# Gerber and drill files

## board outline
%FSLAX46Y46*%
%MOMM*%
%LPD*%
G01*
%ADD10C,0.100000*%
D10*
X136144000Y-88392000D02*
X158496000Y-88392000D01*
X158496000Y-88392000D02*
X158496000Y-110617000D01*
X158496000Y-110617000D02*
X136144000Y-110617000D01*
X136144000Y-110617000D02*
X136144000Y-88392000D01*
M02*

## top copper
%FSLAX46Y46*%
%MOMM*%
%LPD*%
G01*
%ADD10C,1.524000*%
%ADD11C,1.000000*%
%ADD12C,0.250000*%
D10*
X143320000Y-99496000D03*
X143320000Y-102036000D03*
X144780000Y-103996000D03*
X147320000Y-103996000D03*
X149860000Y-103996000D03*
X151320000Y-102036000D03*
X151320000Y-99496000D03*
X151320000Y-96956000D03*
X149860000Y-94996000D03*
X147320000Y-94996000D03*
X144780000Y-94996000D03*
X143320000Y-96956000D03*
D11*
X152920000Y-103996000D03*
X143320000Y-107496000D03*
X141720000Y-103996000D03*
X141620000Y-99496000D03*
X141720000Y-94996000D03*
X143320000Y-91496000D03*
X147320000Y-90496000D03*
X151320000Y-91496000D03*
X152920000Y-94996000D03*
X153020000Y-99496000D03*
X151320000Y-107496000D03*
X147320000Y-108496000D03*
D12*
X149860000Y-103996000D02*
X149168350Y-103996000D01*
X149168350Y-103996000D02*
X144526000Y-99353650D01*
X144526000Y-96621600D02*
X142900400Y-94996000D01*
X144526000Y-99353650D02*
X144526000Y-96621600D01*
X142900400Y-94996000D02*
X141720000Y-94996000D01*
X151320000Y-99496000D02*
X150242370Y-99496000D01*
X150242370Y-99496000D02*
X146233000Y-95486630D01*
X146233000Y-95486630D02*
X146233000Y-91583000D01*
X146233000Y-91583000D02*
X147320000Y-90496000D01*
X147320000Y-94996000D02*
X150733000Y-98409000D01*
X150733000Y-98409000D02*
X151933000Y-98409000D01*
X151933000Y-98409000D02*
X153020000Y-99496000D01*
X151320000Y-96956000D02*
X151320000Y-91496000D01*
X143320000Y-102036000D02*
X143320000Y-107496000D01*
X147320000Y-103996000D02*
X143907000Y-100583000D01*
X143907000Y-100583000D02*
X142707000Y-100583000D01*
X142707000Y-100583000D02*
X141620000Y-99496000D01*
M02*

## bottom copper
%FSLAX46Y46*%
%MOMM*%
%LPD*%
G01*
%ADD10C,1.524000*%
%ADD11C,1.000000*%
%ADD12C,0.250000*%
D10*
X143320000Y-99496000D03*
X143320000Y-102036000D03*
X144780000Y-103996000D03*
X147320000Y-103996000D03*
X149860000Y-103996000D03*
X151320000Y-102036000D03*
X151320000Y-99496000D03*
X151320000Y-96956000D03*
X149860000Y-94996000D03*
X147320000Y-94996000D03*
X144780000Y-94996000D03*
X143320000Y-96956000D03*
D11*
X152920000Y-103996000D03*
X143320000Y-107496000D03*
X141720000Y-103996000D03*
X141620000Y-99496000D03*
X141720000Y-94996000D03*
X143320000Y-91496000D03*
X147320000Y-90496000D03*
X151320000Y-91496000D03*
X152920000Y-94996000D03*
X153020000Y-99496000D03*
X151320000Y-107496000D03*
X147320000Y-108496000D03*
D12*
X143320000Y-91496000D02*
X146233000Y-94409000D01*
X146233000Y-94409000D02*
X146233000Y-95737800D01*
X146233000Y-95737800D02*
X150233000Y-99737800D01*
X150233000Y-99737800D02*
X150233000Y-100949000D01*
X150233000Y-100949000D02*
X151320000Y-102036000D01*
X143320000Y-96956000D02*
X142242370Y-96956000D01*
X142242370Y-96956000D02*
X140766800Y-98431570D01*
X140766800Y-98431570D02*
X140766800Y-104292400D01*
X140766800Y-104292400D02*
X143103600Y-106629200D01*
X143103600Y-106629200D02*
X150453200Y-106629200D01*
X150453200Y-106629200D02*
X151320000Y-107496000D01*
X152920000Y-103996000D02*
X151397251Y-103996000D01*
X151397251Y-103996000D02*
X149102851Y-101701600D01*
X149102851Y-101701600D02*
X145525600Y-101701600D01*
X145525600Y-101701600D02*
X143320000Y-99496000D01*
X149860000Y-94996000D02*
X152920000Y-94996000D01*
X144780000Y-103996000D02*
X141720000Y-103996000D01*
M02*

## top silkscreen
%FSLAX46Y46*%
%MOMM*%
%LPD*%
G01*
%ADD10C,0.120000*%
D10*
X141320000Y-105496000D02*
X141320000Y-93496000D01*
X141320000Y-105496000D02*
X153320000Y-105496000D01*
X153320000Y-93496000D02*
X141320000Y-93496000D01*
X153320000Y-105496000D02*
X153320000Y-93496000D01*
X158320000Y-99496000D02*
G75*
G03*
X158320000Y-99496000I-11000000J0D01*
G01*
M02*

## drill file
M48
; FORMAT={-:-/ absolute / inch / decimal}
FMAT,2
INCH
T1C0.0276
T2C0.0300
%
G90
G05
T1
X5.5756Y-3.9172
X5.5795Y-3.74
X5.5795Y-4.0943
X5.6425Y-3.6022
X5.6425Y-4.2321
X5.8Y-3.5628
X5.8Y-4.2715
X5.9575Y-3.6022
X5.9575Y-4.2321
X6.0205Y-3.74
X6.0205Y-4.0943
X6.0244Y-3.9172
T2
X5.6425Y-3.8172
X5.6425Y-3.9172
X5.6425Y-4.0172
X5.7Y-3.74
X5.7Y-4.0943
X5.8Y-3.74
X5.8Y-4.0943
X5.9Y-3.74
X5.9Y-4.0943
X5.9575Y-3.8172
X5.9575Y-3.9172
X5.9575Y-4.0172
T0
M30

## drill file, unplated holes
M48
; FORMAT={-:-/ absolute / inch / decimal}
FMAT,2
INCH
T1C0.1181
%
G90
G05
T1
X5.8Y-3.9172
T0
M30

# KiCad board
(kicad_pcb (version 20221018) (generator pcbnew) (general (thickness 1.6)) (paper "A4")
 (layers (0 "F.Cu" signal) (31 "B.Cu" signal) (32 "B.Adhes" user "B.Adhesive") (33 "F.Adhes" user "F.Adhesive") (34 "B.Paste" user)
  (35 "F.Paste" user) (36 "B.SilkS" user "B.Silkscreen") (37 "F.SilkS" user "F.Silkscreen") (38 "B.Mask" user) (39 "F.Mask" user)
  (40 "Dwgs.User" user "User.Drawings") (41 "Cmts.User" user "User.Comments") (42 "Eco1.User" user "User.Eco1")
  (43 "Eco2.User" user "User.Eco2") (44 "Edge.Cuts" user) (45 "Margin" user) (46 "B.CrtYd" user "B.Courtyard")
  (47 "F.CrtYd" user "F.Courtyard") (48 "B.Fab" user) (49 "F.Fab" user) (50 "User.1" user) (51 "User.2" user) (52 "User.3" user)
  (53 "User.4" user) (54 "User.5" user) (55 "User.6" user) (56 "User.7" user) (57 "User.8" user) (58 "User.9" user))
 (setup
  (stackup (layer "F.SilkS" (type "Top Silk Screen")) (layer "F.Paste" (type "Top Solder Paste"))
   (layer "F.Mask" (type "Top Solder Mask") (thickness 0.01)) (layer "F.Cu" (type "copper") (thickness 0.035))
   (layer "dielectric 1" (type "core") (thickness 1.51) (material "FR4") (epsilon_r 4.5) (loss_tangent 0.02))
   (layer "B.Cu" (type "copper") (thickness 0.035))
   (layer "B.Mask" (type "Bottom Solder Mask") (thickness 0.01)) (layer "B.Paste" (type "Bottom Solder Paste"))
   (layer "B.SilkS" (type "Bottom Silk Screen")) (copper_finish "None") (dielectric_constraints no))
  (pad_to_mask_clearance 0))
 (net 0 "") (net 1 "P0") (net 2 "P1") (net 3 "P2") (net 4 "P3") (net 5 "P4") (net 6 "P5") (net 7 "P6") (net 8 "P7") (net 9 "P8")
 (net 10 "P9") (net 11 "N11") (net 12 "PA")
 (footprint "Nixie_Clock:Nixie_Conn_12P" (layer "F.Cu") (at 147.32 99.496)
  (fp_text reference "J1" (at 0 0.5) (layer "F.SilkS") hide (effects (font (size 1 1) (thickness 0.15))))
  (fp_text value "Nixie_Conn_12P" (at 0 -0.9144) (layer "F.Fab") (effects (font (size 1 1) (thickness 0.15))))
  (fp_line (start -6 6) (end -6 -6) (stroke (width 0.12) (type solid)) (layer "F.SilkS"))
  (fp_line (start -6 6) (end 6 6) (stroke (width 0.12) (type solid)) (layer "F.SilkS"))
  (fp_line (start 6 -6) (end -6 -6) (stroke (width 0.12) (type solid)) (layer "F.SilkS"))
  (fp_line (start 6 6) (end 6 -6) (stroke (width 0.12) (type solid)) (layer "F.SilkS"))
  (pad "0" thru_hole circle (at -4 0) (size 1.524 1.524) (drill 0.762) (layers "*.Cu" "*.Mask") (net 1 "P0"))
  (pad "1" thru_hole circle (at -4 2.54) (size 1.524 1.524) (drill 0.762) (layers "*.Cu" "*.Mask") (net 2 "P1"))
  (pad "2" thru_hole circle (at -2.54 4.5) (size 1.524 1.524) (drill 0.762) (layers "*.Cu" "*.Mask") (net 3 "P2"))
  (pad "3" thru_hole circle (at 0 4.5) (size 1.524 1.524) (drill 0.762) (layers "*.Cu" "*.Mask") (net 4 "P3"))
  (pad "4" thru_hole circle (at 2.54 4.5) (size 1.524 1.524) (drill 0.762) (layers "*.Cu" "*.Mask") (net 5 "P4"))
  (pad "5" thru_hole circle (at 4 2.54) (size 1.524 1.524) (drill 0.762) (layers "*.Cu" "*.Mask") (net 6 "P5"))
  (pad "6" thru_hole circle (at 4 0) (size 1.524 1.524) (drill 0.762) (layers "*.Cu" "*.Mask") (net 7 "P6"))
  (pad "7" thru_hole circle (at 4 -2.54) (size 1.524 1.524) (drill 0.762) (layers "*.Cu" "*.Mask") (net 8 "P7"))
  (pad "8" thru_hole circle (at 2.54 -4.5) (size 1.524 1.524) (drill 0.762) (layers "*.Cu" "*.Mask") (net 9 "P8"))
  (pad "9" thru_hole circle (at 0 -4.5) (size 1.524 1.524) (drill 0.762) (layers "*.Cu" "*.Mask") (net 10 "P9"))
  (pad "10" thru_hole circle (at -2.54 -4.5) (size 1.524 1.524) (drill 0.762) (layers "*.Cu" "*.Mask") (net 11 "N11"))
  (pad "A" thru_hole circle (at -4 -2.54) (size 1.524 1.524) (drill 0.762) (layers "*.Cu" "*.Mask") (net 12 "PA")))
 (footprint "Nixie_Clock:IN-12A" (layer "F.Cu") (at 147.32 99.496)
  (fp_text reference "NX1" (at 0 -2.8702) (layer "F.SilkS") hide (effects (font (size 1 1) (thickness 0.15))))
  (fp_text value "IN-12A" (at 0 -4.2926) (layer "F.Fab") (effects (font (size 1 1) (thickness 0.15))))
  (fp_circle (center 0 0) (end 11 0) (stroke (width 0.12) (type solid)) (fill none) (layer "F.SilkS"))
  (pad "" np_thru_hole circle (at 0 0) (size 3 3) (drill 3) (layers "*.Cu" "*.Mask"))
  (pad "0" thru_hole circle (at 5.6 4.5) (size 1 1) (drill 0.7) (layers "*.Cu" "*.Mask") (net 1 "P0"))
  (pad "1" thru_hole circle (at -4 8) (size 1 1) (drill 0.7) (layers "*.Cu" "*.Mask") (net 2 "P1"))
  (pad "2" thru_hole circle (at -5.6 4.5) (size 1 1) (drill 0.7) (layers "*.Cu" "*.Mask") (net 3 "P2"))
  (pad "3" thru_hole circle (at -5.7 0) (size 1 1) (drill 0.7) (layers "*.Cu" "*.Mask") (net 4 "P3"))
  (pad "4" thru_hole circle (at -5.6 -4.5) (size 1 1) (drill 0.7) (layers "*.Cu" "*.Mask") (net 5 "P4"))
  (pad "5" thru_hole circle (at -4 -8) (size 1 1) (drill 0.7) (layers "*.Cu" "*.Mask") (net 6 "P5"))
  (pad "6" thru_hole circle (at 0 -9) (size 1 1) (drill 0.7) (layers "*.Cu" "*.Mask") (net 7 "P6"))
  (pad "7" thru_hole circle (at 4 -8) (size 1 1) (drill 0.7) (layers "*.Cu" "*.Mask") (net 8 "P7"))
  (pad "8" thru_hole circle (at 5.6 -4.5) (size 1 1) (drill 0.7) (layers "*.Cu" "*.Mask") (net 9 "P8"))
  (pad "9" thru_hole circle (at 5.7 0) (size 1 1) (drill 0.7) (layers "*.Cu" "*.Mask") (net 10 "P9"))
  (pad "A" thru_hole circle (at 4 8) (size 1 1) (drill 0.7) (layers "*.Cu" "*.Mask") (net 12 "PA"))
  (pad "DP" thru_hole circle (at 0 9) (size 1 1) (drill 0.7) (layers "*.Cu" "*.Mask")))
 (gr_rect (start 136.144 88.392) (end 158.496 110.617) (stroke (width 0.1) (type default)) (fill none) (layer "Edge.Cuts"))
 (segment (start 149.102851 101.7016) (end 145.5256 101.7016) (width 0.25) (layer "B.Cu") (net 1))
 (segment (start 145.5256 101.7016) (end 143.32 99.496) (width 0.25) (layer "B.Cu") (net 1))
 (segment (start 152.92 103.996) (end 151.397251 103.996) (width 0.25) (layer "B.Cu") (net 1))
 (segment (start 151.397251 103.996) (end 149.102851 101.7016) (width 0.25) (layer "B.Cu") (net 1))
 (segment (start 143.32 102.036) (end 143.32 107.496) (width 0.25) (layer "F.Cu") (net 2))
 (segment (start 144.78 103.996) (end 141.72 103.996) (width 0.25) (layer "B.Cu") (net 3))
 (segment (start 143.907 100.583) (end 142.707 100.583) (width 0.25) (layer "F.Cu") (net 4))
 (segment (start 147.32 103.996) (end 143.907 100.583) (width 0.25) (layer "F.Cu") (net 4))
 (segment (start 142.707 100.583) (end 141.62 99.496) (width 0.25) (layer "F.Cu") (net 4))
 (segment (start 144.526 99.35365) (end 144.526 96.6216) (width 0.25) (layer "F.Cu") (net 5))
 (segment (start 149.16835 103.996) (end 144.526 99.35365) (width 0.25) (layer "F.Cu") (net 5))
 (segment (start 149.86 103.996) (end 149.16835 103.996) (width 0.25) (layer "F.Cu") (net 5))
 (segment (start 144.526 96.6216) (end 142.9004 94.996) (width 0.25) (layer "F.Cu") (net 5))
 (segment (start 142.9004 94.996) (end 141.72 94.996) (width 0.25) (layer "F.Cu") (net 5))
 (segment (start 150.233 100.949) (end 151.32 102.036) (width 0.25) (layer "B.Cu") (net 6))
 (segment (start 146.233 94.409) (end 146.233 95.7378) (width 0.25) (layer "B.Cu") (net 6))
 (segment (start 143.32 91.496) (end 146.233 94.409) (width 0.25) (layer "B.Cu") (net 6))
 (segment (start 150.233 99.7378) (end 150.233 100.949) (width 0.25) (layer "B.Cu") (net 6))
 (segment (start 146.233 95.7378) (end 150.233 99.7378) (width 0.25) (layer "B.Cu") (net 6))
 (segment (start 146.233 91.583) (end 147.32 90.496) (width 0.25) (layer "F.Cu") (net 7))
 (segment (start 146.233 95.48663) (end 146.233 91.583) (width 0.25) (layer "F.Cu") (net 7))
 (segment (start 150.24237 99.496) (end 146.233 95.48663) (width 0.25) (layer "F.Cu") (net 7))
 (segment (start 151.32 99.496) (end 150.24237 99.496) (width 0.25) (layer "F.Cu") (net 7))
 (segment (start 151.32 96.956) (end 151.32 91.496) (width 0.25) (layer "F.Cu") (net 8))
 (segment (start 149.86 94.996) (end 152.92 94.996) (width 0.25) (layer "B.Cu") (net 9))
 (segment (start 150.733 98.409) (end 151.933 98.409) (width 0.25) (layer "F.Cu") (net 10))
 (segment (start 151.933 98.409) (end 153.02 99.496) (width 0.25) (layer "F.Cu") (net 10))
 (segment (start 147.32 94.996) (end 150.733 98.409) (width 0.25) (layer "F.Cu") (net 10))
 (segment (start 140.7668 98.43157) (end 140.7668 104.2924) (width 0.25) (layer "B.Cu") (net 12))
 (segment (start 142.24237 96.956) (end 140.7668 98.43157) (width 0.25) (layer "B.Cu") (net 12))
 (segment (start 143.32 96.956) (end 142.24237 96.956) (width 0.25) (layer "B.Cu") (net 12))
 (segment (start 150.4532 106.6292) (end 151.32 107.496) (width 0.25) (layer "B.Cu") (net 12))
 (segment (start 143.1036 106.6292) (end 150.4532 106.6292) (width 0.25) (layer "B.Cu") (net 12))
 (segment (start 140.7668 104.2924) (end 143.1036 106.6292) (width 0.25) (layer "B.Cu") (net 12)))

